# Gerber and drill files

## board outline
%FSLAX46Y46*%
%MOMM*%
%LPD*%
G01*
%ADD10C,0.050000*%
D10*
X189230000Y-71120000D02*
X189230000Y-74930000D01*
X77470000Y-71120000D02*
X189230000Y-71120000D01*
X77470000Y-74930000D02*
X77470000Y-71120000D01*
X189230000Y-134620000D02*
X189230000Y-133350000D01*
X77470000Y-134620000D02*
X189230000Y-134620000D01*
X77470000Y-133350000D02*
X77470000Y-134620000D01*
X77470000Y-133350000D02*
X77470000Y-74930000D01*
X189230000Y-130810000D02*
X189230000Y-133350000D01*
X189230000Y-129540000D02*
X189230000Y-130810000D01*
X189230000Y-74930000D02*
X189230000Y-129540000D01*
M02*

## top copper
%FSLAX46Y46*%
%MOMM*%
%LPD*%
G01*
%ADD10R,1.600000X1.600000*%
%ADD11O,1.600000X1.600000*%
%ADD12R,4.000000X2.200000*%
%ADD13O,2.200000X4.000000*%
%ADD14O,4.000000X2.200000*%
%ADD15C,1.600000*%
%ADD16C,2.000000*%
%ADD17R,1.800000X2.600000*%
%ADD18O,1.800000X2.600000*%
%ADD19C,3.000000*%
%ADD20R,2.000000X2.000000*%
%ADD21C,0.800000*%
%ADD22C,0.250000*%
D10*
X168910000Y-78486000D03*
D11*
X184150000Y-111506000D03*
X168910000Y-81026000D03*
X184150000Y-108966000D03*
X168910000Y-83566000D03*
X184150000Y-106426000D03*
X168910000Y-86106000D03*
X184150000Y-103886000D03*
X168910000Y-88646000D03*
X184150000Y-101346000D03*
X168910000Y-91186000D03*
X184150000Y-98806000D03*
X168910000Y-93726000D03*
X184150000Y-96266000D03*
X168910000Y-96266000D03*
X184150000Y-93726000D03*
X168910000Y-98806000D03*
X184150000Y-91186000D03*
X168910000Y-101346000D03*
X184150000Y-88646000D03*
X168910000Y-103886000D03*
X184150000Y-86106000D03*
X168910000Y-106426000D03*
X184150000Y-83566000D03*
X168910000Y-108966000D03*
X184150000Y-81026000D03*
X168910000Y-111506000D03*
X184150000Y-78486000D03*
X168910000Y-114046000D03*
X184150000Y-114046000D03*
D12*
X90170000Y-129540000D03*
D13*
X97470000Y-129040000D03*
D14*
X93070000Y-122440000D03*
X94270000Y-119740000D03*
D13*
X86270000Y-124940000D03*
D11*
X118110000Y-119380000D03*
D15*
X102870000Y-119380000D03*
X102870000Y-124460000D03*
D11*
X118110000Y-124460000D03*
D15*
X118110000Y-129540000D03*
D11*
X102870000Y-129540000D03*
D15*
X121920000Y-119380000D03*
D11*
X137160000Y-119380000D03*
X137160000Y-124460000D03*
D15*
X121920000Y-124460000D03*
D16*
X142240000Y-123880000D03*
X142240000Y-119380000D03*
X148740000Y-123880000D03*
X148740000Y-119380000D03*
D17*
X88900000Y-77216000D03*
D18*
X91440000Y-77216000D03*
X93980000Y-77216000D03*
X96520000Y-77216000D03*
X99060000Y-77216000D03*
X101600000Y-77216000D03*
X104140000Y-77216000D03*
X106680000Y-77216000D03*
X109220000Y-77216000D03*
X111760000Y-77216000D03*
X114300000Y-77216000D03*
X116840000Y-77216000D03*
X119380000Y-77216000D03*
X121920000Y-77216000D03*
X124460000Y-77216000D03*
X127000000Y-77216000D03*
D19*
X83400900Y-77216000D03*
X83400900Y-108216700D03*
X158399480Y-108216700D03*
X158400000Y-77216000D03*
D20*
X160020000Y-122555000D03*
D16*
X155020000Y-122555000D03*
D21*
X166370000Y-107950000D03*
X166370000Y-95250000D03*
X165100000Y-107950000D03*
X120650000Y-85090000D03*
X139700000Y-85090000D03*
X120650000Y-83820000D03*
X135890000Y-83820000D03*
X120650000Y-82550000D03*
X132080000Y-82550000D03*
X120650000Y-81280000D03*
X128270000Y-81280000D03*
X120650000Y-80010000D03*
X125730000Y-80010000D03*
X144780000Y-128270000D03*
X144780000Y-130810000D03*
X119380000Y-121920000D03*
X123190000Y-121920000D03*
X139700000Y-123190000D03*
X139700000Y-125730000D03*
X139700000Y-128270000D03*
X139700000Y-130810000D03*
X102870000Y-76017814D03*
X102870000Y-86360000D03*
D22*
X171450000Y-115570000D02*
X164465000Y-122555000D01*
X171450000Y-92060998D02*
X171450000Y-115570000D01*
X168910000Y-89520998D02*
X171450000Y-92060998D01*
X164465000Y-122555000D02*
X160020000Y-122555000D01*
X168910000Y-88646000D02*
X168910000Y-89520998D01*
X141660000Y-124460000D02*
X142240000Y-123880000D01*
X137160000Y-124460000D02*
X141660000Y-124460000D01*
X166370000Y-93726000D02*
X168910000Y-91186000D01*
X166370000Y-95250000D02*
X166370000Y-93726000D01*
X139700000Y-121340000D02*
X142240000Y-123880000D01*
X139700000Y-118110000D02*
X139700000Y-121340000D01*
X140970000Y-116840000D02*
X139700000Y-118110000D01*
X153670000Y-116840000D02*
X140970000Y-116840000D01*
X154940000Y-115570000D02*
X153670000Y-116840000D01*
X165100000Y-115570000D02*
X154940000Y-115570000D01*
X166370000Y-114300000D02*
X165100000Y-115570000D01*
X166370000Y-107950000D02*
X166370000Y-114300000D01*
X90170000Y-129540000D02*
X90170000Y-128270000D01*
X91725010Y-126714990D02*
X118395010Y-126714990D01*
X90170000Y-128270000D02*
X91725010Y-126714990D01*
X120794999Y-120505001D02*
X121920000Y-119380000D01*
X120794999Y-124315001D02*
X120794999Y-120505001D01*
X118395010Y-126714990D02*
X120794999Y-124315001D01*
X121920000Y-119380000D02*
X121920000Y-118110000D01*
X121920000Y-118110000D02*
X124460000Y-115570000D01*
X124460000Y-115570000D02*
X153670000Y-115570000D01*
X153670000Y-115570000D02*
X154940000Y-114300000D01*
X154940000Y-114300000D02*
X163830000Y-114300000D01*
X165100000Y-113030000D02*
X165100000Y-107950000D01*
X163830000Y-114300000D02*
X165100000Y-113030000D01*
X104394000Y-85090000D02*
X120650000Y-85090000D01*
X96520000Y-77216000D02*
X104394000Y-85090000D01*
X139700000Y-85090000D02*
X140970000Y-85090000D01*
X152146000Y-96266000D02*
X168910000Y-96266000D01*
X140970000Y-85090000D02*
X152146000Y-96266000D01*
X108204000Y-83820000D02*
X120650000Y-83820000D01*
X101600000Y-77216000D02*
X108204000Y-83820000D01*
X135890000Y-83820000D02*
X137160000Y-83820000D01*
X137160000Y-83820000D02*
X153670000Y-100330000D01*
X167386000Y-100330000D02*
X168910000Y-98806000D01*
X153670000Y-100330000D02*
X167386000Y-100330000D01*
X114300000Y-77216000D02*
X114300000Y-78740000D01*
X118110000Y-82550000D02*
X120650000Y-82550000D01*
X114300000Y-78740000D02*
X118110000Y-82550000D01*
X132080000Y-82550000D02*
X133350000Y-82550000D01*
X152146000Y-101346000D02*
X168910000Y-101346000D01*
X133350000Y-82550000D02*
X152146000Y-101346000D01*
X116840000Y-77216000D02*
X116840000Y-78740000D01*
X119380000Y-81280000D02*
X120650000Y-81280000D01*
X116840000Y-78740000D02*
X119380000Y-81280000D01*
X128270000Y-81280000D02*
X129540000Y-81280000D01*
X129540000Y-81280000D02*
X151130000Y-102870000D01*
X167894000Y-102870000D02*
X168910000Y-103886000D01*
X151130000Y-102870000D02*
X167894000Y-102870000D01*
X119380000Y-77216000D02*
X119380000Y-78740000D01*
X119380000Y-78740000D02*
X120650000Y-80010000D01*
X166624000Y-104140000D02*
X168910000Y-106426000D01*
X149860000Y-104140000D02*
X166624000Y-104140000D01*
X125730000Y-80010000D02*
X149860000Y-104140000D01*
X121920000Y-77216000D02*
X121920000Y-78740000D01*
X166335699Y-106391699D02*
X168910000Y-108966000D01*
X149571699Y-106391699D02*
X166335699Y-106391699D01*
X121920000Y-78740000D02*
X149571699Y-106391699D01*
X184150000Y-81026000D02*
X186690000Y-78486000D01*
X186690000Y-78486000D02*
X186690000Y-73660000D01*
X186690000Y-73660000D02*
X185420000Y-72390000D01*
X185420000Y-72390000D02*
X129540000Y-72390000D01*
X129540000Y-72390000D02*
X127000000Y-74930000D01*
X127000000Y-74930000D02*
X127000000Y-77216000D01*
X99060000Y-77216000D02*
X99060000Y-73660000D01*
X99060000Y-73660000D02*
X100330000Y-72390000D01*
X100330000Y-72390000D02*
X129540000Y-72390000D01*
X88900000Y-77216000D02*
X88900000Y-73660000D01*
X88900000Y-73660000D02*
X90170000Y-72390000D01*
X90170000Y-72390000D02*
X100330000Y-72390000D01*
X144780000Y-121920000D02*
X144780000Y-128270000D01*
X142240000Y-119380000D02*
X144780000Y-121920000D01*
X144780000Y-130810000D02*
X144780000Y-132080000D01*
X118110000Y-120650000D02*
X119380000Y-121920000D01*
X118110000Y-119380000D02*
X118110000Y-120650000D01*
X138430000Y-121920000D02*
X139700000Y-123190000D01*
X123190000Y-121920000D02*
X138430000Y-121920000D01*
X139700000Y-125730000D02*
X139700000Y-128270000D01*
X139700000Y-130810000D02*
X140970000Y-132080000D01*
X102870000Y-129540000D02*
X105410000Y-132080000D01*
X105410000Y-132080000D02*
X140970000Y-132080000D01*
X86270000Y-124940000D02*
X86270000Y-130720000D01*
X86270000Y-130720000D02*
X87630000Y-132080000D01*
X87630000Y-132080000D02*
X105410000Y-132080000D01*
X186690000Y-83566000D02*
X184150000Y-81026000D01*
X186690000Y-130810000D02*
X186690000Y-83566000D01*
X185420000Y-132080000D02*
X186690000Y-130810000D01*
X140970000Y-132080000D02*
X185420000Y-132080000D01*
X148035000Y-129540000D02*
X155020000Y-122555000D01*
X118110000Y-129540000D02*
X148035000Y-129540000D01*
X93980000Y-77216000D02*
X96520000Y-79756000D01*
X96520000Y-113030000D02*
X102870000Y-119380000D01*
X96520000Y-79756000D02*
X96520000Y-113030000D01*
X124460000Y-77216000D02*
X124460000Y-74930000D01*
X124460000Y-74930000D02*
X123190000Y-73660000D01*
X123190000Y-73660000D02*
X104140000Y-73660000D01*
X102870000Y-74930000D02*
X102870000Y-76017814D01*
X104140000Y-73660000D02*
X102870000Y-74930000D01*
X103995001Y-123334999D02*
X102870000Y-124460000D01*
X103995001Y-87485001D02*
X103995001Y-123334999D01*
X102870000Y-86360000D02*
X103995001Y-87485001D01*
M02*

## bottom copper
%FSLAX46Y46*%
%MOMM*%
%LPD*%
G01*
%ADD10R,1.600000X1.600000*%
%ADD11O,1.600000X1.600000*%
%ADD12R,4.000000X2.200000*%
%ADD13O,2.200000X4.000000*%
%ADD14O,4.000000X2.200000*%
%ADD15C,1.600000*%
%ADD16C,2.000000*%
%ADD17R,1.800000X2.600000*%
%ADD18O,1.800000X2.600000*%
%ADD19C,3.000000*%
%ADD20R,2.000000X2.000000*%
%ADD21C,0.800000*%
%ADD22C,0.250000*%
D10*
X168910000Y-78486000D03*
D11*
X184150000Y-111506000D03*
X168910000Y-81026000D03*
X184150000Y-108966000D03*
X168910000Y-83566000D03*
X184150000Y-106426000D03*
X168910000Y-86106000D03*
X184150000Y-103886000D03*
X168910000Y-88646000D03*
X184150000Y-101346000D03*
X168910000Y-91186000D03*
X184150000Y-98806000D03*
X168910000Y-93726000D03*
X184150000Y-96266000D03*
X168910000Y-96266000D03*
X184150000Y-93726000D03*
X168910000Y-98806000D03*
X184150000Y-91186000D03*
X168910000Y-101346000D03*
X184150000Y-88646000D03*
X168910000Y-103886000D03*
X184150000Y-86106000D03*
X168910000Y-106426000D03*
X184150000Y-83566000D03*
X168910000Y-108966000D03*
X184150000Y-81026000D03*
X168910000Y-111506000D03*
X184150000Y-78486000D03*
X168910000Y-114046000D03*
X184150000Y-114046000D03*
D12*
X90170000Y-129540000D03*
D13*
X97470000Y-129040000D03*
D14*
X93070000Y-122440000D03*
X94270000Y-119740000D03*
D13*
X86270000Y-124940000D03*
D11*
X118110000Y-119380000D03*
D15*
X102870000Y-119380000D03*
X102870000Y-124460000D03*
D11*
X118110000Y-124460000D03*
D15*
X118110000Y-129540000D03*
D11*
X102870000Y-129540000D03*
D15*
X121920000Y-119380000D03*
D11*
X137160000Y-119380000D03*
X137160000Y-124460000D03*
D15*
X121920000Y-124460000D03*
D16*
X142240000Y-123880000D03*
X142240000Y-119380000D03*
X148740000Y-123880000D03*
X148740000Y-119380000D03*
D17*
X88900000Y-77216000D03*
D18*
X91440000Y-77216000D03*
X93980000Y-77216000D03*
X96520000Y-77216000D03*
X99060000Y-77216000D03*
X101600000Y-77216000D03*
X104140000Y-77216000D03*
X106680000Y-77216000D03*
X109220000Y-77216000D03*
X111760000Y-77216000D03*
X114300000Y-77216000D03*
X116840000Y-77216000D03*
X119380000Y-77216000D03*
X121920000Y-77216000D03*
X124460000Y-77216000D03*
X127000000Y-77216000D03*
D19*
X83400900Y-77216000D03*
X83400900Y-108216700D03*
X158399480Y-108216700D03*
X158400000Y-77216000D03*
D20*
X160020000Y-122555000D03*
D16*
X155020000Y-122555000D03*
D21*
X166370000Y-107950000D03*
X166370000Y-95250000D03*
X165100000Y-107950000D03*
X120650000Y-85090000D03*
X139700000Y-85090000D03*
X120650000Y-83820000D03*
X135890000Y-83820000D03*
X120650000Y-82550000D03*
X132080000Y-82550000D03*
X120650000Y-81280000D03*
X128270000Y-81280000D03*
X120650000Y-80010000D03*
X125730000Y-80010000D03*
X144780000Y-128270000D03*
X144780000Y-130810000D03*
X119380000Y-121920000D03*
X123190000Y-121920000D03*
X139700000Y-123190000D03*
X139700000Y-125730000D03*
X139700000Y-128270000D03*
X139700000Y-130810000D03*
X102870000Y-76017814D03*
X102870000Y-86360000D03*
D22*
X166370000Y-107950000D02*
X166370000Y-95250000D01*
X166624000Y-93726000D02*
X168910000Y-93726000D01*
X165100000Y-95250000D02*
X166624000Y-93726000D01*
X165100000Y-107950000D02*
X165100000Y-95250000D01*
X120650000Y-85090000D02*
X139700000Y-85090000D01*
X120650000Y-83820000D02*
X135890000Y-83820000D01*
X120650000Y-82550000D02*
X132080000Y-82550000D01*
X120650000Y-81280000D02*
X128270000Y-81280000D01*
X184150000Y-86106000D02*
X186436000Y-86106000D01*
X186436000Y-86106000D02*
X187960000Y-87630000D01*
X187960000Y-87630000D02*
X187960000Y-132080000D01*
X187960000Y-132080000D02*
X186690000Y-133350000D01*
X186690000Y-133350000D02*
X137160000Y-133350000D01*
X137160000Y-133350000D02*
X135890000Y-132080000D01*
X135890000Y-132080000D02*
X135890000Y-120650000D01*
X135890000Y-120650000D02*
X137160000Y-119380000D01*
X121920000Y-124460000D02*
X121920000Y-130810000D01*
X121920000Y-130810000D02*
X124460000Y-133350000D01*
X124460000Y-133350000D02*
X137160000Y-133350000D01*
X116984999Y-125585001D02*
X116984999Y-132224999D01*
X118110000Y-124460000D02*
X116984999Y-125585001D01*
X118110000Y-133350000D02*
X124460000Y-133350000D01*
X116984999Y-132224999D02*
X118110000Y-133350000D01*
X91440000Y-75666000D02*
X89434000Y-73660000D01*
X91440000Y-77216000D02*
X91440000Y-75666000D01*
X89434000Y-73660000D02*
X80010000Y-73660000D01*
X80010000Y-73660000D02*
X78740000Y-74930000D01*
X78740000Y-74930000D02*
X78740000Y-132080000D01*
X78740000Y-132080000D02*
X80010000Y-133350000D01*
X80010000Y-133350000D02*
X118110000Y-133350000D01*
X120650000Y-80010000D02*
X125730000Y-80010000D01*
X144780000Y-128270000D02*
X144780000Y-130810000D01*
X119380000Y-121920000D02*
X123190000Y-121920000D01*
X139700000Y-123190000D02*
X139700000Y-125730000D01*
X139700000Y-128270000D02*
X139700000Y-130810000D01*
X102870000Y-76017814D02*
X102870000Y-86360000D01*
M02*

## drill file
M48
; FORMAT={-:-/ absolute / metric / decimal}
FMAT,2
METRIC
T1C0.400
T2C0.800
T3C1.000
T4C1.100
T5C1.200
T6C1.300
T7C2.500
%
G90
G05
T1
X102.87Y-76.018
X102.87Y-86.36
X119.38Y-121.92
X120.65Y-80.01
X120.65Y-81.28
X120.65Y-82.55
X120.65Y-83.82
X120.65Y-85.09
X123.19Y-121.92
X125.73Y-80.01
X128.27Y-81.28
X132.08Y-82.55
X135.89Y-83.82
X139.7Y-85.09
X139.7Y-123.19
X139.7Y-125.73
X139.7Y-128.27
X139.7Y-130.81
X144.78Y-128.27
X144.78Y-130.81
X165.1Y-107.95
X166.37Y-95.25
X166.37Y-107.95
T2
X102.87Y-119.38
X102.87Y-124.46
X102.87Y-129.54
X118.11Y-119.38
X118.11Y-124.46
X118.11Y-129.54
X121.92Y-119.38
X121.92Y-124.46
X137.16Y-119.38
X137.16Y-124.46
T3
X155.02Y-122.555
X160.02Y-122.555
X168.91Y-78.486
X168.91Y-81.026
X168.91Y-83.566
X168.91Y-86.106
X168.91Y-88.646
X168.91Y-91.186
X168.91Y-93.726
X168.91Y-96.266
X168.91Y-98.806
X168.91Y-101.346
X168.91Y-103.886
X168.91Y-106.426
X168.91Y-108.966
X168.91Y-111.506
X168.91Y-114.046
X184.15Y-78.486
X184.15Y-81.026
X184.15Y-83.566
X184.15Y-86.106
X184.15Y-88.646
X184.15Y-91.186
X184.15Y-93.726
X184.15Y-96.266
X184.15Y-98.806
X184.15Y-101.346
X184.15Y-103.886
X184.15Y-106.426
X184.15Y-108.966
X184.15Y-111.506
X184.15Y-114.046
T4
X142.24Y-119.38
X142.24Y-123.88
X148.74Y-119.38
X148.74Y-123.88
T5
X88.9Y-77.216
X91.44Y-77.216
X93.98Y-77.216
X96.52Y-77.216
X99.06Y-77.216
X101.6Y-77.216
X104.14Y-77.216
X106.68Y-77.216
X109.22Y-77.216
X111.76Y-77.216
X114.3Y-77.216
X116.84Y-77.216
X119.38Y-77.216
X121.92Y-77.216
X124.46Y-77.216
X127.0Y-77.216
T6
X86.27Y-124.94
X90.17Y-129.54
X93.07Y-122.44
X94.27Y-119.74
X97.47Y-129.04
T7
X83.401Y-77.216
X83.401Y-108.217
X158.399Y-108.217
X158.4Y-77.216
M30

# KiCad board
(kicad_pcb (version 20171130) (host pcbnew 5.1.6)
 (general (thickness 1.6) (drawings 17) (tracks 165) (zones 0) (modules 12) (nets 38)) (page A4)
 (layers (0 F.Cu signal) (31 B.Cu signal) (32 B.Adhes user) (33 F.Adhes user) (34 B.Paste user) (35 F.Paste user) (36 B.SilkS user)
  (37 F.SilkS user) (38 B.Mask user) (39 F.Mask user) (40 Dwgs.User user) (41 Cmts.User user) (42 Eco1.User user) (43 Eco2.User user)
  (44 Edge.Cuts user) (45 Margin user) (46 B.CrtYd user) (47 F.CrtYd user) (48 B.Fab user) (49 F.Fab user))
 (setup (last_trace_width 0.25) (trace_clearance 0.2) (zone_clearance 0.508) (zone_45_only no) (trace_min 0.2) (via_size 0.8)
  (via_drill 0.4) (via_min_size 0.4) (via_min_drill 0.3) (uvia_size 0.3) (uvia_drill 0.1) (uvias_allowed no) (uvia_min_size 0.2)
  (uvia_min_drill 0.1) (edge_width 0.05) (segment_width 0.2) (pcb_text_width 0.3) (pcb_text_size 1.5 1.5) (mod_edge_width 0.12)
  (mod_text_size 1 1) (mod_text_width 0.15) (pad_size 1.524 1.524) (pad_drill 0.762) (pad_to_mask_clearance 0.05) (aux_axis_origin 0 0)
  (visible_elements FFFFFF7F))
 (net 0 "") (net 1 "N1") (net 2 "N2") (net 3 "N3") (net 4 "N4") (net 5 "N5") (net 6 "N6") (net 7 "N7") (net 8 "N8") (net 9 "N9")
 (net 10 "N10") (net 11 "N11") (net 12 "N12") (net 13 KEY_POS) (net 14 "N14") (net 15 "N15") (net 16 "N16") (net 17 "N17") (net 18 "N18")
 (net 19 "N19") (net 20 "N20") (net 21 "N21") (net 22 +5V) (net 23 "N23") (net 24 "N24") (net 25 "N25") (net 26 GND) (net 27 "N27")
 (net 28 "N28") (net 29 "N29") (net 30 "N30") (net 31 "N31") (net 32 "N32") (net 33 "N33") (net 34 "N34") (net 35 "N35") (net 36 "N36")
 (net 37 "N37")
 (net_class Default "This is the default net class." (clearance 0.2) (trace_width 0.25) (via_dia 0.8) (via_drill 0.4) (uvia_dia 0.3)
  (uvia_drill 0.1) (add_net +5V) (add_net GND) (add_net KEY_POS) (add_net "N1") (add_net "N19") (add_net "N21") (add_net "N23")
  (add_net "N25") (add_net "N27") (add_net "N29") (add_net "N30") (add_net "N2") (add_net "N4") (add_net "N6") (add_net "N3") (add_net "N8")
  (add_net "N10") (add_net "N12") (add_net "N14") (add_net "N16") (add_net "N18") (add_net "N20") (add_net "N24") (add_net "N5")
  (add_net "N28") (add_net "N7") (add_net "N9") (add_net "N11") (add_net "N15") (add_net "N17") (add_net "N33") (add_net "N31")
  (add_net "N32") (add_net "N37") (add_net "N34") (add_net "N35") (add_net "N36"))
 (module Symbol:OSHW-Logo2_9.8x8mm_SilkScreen (layer F.Cu) (at 181.102 124.968)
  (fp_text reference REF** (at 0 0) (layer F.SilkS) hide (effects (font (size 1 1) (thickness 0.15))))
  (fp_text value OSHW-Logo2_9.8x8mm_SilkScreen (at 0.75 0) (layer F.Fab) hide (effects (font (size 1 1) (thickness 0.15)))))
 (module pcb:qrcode (layer F.Cu) (at 172.466 125.222)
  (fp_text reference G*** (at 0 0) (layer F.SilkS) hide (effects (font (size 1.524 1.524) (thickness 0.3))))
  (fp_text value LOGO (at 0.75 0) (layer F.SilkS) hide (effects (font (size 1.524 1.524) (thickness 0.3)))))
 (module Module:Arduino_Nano (layer F.Cu) (at 168.91 78.486)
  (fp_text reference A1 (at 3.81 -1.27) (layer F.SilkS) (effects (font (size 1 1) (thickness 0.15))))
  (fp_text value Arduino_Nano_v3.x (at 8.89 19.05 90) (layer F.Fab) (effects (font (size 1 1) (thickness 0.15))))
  (pad 1 thru_hole rect (at 0 0) (size 1.6 1.6) (drill 1) (layers *.Cu *.Mask) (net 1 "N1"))
  (pad 17 thru_hole oval (at 15.24 33.02) (size 1.6 1.6) (drill 1) (layers *.Cu *.Mask) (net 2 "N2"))
  (pad 2 thru_hole oval (at 0 2.54) (size 1.6 1.6) (drill 1) (layers *.Cu *.Mask) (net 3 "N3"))
  (pad 18 thru_hole oval (at 15.24 30.48) (size 1.6 1.6) (drill 1) (layers *.Cu *.Mask) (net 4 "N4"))
  (pad 3 thru_hole oval (at 0 5.08) (size 1.6 1.6) (drill 1) (layers *.Cu *.Mask) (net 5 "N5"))
  (pad 19 thru_hole oval (at 15.24 27.94) (size 1.6 1.6) (drill 1) (layers *.Cu *.Mask) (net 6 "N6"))
  (pad 4 thru_hole oval (at 0 7.62) (size 1.6 1.6) (drill 1) (layers *.Cu *.Mask) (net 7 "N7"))
  (pad 20 thru_hole oval (at 15.24 25.4) (size 1.6 1.6) (drill 1) (layers *.Cu *.Mask) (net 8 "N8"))
  (pad 5 thru_hole oval (at 0 10.16) (size 1.6 1.6) (drill 1) (layers *.Cu *.Mask) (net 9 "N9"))
  (pad 21 thru_hole oval (at 15.24 22.86) (size 1.6 1.6) (drill 1) (layers *.Cu *.Mask) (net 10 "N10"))
  (pad 6 thru_hole oval (at 0 12.7) (size 1.6 1.6) (drill 1) (layers *.Cu *.Mask) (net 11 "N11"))
  (pad 22 thru_hole oval (at 15.24 20.32) (size 1.6 1.6) (drill 1) (layers *.Cu *.Mask) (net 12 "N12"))
  (pad 7 thru_hole oval (at 0 15.24) (size 1.6 1.6) (drill 1) (layers *.Cu *.Mask) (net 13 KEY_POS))
  (pad 23 thru_hole oval (at 15.24 17.78) (size 1.6 1.6) (drill 1) (layers *.Cu *.Mask) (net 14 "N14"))
  (pad 8 thru_hole oval (at 0 17.78) (size 1.6 1.6) (drill 1) (layers *.Cu *.Mask) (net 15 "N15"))
  (pad 24 thru_hole oval (at 15.24 15.24) (size 1.6 1.6) (drill 1) (layers *.Cu *.Mask) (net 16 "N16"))
  (pad 9 thru_hole oval (at 0 20.32) (size 1.6 1.6) (drill 1) (layers *.Cu *.Mask) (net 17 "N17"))
  (pad 25 thru_hole oval (at 15.24 12.7) (size 1.6 1.6) (drill 1) (layers *.Cu *.Mask) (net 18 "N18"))
  (pad 10 thru_hole oval (at 0 22.86) (size 1.6 1.6) (drill 1) (layers *.Cu *.Mask) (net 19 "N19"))
  (pad 26 thru_hole oval (at 15.24 10.16) (size 1.6 1.6) (drill 1) (layers *.Cu *.Mask) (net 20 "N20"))
  (pad 11 thru_hole oval (at 0 25.4) (size 1.6 1.6) (drill 1) (layers *.Cu *.Mask) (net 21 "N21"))
  (pad 27 thru_hole oval (at 15.24 7.62) (size 1.6 1.6) (drill 1) (layers *.Cu *.Mask) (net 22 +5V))
  (pad 12 thru_hole oval (at 0 27.94) (size 1.6 1.6) (drill 1) (layers *.Cu *.Mask) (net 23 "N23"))
  (pad 28 thru_hole oval (at 15.24 5.08) (size 1.6 1.6) (drill 1) (layers *.Cu *.Mask) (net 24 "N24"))
  (pad 13 thru_hole oval (at 0 30.48) (size 1.6 1.6) (drill 1) (layers *.Cu *.Mask) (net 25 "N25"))
  (pad 29 thru_hole oval (at 15.24 2.54) (size 1.6 1.6) (drill 1) (layers *.Cu *.Mask) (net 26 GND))
  (pad 14 thru_hole oval (at 0 33.02) (size 1.6 1.6) (drill 1) (layers *.Cu *.Mask) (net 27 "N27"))
  (pad 30 thru_hole oval (at 15.24 0) (size 1.6 1.6) (drill 1) (layers *.Cu *.Mask) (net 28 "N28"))
  (pad 15 thru_hole oval (at 0 35.56) (size 1.6 1.6) (drill 1) (layers *.Cu *.Mask) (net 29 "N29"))
  (pad 16 thru_hole oval (at 15.24 35.56) (size 1.6 1.6) (drill 1) (layers *.Cu *.Mask) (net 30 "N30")))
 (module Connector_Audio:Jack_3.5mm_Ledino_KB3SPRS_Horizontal (layer F.Cu) (at 90.17 129.54)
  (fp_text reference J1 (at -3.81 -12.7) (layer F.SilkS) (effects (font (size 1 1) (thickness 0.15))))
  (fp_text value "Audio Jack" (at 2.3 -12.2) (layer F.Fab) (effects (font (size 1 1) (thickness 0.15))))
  (pad T thru_hole rect (at 0 0) (size 4 2.2) (drill 1.3) (layers *.Cu *.Mask) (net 13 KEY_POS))
  (pad TN thru_hole oval (at 7.3 -0.5 90) (size 4 2.2) (drill 1.3) (layers *.Cu *.Mask))
  (pad RN thru_hole oval (at 2.9 -7.1) (size 4 2.2) (drill 1.3) (layers *.Cu *.Mask))
  (pad R thru_hole oval (at 4.1 -9.8) (size 4 2.2) (drill 1.3) (layers *.Cu *.Mask))
  (pad S thru_hole oval (at -3.9 -4.6) (size 2.2 4) (drill 1.3) (layers *.Cu *.Mask) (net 26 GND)))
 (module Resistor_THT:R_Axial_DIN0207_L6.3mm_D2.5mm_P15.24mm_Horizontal (layer F.Cu) (at 102.87 119.38)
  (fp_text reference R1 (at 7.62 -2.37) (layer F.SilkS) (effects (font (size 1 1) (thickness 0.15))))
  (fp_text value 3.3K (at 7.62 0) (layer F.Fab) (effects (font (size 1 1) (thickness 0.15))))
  (pad 2 thru_hole oval (at 15.24 0) (size 1.6 1.6) (drill 0.8) (layers *.Cu *.Mask) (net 26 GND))
  (pad 1 thru_hole circle (at 0 0) (size 1.6 1.6) (drill 0.8) (layers *.Cu *.Mask) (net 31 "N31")))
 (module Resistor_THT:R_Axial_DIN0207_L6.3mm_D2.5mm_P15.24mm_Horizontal (layer F.Cu) (at 102.87 124.46)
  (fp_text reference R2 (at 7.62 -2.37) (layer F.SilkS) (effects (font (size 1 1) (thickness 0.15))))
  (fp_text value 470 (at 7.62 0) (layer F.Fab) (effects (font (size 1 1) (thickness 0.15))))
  (pad 1 thru_hole circle (at 0 0) (size 1.6 1.6) (drill 0.8) (layers *.Cu *.Mask) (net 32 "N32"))
  (pad 2 thru_hole oval (at 15.24 0) (size 1.6 1.6) (drill 0.8) (layers *.Cu *.Mask) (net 22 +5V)))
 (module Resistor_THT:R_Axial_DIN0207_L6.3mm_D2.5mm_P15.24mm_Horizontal (layer F.Cu) (at 118.11 129.54 180)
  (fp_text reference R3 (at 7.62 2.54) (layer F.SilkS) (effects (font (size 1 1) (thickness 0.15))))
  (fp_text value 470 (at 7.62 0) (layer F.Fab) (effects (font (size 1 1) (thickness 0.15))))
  (pad 1 thru_hole circle (at 0 0 180) (size 1.6 1.6) (drill 0.8) (layers *.Cu *.Mask) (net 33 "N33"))
  (pad 2 thru_hole oval (at 15.24 0 180) (size 1.6 1.6) (drill 0.8) (layers *.Cu *.Mask) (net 26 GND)))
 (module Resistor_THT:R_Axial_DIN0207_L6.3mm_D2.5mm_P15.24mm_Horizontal (layer F.Cu) (at 121.92 119.38)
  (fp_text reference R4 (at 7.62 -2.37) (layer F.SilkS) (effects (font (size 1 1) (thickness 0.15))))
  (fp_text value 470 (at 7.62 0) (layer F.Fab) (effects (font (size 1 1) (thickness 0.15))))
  (pad 1 thru_hole circle (at 0 0) (size 1.6 1.6) (drill 0.8) (layers *.Cu *.Mask) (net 13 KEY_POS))
  (pad 2 thru_hole oval (at 15.24 0) (size 1.6 1.6) (drill 0.8) (layers *.Cu *.Mask) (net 22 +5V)))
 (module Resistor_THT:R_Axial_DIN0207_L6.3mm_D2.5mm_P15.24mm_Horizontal (layer F.Cu) (at 121.92 124.46)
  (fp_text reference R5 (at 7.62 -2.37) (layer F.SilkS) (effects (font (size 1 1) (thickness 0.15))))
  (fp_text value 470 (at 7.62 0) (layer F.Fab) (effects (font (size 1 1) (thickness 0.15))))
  (pad 2 thru_hole oval (at 15.24 0) (size 1.6 1.6) (drill 0.8) (layers *.Cu *.Mask) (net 11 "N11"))
  (pad 1 thru_hole circle (at 0 0) (size 1.6 1.6) (drill 0.8) (layers *.Cu *.Mask) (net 22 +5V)))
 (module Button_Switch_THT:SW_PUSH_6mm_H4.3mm (layer F.Cu) (at 142.24 119.38)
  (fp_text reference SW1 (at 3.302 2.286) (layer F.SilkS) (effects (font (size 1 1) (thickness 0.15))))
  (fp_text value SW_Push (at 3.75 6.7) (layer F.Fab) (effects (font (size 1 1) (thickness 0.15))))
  (pad 2 thru_hole circle (at 0 4.5 90) (size 2 2) (drill 1.1) (layers *.Cu *.Mask) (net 11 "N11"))
  (pad 1 thru_hole circle (at 0 0 90) (size 2 2) (drill 1.1) (layers *.Cu *.Mask) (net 26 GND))
  (pad 2 thru_hole circle (at 6.5 4.5 90) (size 2 2) (drill 1.1) (layers *.Cu *.Mask) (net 11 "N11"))
  (pad 1 thru_hole circle (at 6.5 0 90) (size 2 2) (drill 1.1) (layers *.Cu *.Mask) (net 26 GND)))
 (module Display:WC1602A (layer F.Cu) (at 88.9 77.216)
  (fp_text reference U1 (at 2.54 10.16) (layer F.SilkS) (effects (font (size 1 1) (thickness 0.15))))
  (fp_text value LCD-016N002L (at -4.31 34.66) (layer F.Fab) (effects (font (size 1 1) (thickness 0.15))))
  (pad 1 thru_hole rect (at 0 0) (size 1.8 2.6) (drill 1.2) (layers *.Cu *.Mask) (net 26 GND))
  (pad 2 thru_hole oval (at 2.54 0) (size 1.8 2.6) (drill 1.2) (layers *.Cu *.Mask) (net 22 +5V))
  (pad 3 thru_hole oval (at 5.08 0) (size 1.8 2.6) (drill 1.2) (layers *.Cu *.Mask) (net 31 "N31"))
  (pad 4 thru_hole oval (at 7.62 0) (size 1.8 2.6) (drill 1.2) (layers *.Cu *.Mask) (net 15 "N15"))
  (pad 5 thru_hole oval (at 10.16 0) (size 1.8 2.6) (drill 1.2) (layers *.Cu *.Mask) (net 26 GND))
  (pad 6 thru_hole oval (at 12.7 0) (size 1.8 2.6) (drill 1.2) (layers *.Cu *.Mask) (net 17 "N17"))
  (pad 7 thru_hole oval (at 15.24 0) (size 1.8 2.6) (drill 1.2) (layers *.Cu *.Mask) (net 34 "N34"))
  (pad 8 thru_hole oval (at 17.78 0) (size 1.8 2.6) (drill 1.2) (layers *.Cu *.Mask) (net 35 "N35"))
  (pad 9 thru_hole oval (at 20.32 0) (size 1.8 2.6) (drill 1.2) (layers *.Cu *.Mask) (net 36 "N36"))
  (pad 10 thru_hole oval (at 22.86 0) (size 1.8 2.6) (drill 1.2) (layers *.Cu *.Mask) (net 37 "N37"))
  (pad 11 thru_hole oval (at 25.4 0) (size 1.8 2.6) (drill 1.2) (layers *.Cu *.Mask) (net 19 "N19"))
  (pad 12 thru_hole oval (at 27.94 0) (size 1.8 2.6) (drill 1.2) (layers *.Cu *.Mask) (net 21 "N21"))
  (pad 13 thru_hole oval (at 30.48 0) (size 1.8 2.6) (drill 1.2) (layers *.Cu *.Mask) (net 23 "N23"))
  (pad 14 thru_hole oval (at 33.02 0) (size 1.8 2.6) (drill 1.2) (layers *.Cu *.Mask) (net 25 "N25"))
  (pad 15 thru_hole oval (at 35.56 0) (size 1.8 2.6) (drill 1.2) (layers *.Cu *.Mask) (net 32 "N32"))
  (pad 16 thru_hole oval (at 38.1 0) (size 1.8 2.6) (drill 1.2) (layers *.Cu *.Mask) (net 26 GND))
  (pad "" thru_hole circle (at -5.4991 0) (size 3 3) (drill 2.5) (layers *.Cu *.Mask))
  (pad "" thru_hole circle (at -5.4991 31.0007) (size 3 3) (drill 2.5) (layers *.Cu *.Mask))
  (pad "" thru_hole circle (at 69.49948 31.0007) (size 3 3) (drill 2.5) (layers *.Cu *.Mask))
  (pad "" thru_hole circle (at 69.5 0) (size 3 3) (drill 2.5) (layers *.Cu *.Mask)))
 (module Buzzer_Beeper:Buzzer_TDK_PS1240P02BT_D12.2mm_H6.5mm (layer F.Cu) (at 160.02 122.555 180)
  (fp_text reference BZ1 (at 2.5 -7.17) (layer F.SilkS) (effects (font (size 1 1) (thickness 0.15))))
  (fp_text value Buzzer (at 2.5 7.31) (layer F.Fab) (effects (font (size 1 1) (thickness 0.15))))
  (pad 1 thru_hole rect (at 0 0 180) (size 2 2) (drill 1) (layers *.Cu *.Mask) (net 9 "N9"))
  (pad 2 thru_hole circle (at 5 0 180) (size 2 2) (drill 1) (layers *.Cu *.Mask) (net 33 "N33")))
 (gr_line (start 189.23 71.12) (end 189.23 74.93) (layer Edge.Cuts) (width 0.05))
 (gr_line (start 77.47 71.12) (end 189.23 71.12) (layer Edge.Cuts) (width 0.05))
 (gr_line (start 77.47 74.93) (end 77.47 71.12) (layer Edge.Cuts) (width 0.05))
 (gr_line (start 189.23 134.62) (end 189.23 133.35) (layer Edge.Cuts) (width 0.05))
 (gr_line (start 77.47 134.62) (end 189.23 134.62) (layer Edge.Cuts) (width 0.05))
 (gr_line (start 77.47 133.35) (end 77.47 134.62) (layer Edge.Cuts) (width 0.05))
 (gr_line (start 77.47 133.35) (end 77.47 74.93) (layer Edge.Cuts) (width 0.05))
 (gr_line (start 189.23 130.81) (end 189.23 133.35) (layer Edge.Cuts) (width 0.05))
 (gr_line (start 189.23 129.54) (end 189.23 130.81) (layer Edge.Cuts) (width 0.05))
 (gr_line (start 189.23 74.93) (end 189.23 129.54) (layer Edge.Cuts) (width 0.05))
 (segment (start 171.45 115.57) (end 164.465 122.555) (width 0.25) (layer F.Cu) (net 9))
 (segment (start 171.45 92.060998) (end 171.45 115.57) (width 0.25) (layer F.Cu) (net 9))
 (segment (start 168.91 89.520998) (end 171.45 92.060998) (width 0.25) (layer F.Cu) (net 9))
 (segment (start 164.465 122.555) (end 160.02 122.555) (width 0.25) (layer F.Cu) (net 9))
 (segment (start 168.91 88.646) (end 168.91 89.520998) (width 0.25) (layer F.Cu) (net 9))
 (segment (start 141.66 124.46) (end 142.24 123.88) (width 0.25) (layer F.Cu) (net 11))
 (segment (start 137.16 124.46) (end 141.66 124.46) (width 0.25) (layer F.Cu) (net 11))
 (via (at 166.37 107.95) (size 0.8) (drill 0.4) (layers F.Cu B.Cu) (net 11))
 (via (at 166.37 95.25) (size 0.8) (drill 0.4) (layers F.Cu B.Cu) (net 11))
 (segment (start 166.37 107.95) (end 166.37 95.25) (width 0.25) (layer B.Cu) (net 11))
 (segment (start 166.37 93.726) (end 168.91 91.186) (width 0.25) (layer F.Cu) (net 11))
 (segment (start 166.37 95.25) (end 166.37 93.726) (width 0.25) (layer F.Cu) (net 11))
 (segment (start 139.7 121.34) (end 142.24 123.88) (width 0.25) (layer F.Cu) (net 11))
 (segment (start 139.7 118.11) (end 139.7 121.34) (width 0.25) (layer F.Cu) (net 11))
 (segment (start 140.97 116.84) (end 139.7 118.11) (width 0.25) (layer F.Cu) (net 11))
 (segment (start 153.67 116.84) (end 140.97 116.84) (width 0.25) (layer F.Cu) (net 11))
 (segment (start 154.94 115.57) (end 153.67 116.84) (width 0.25) (layer F.Cu) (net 11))
 (segment (start 165.1 115.57) (end 154.94 115.57) (width 0.25) (layer F.Cu) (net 11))
 (segment (start 166.37 114.3) (end 165.1 115.57) (width 0.25) (layer F.Cu) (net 11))
 (segment (start 166.37 107.95) (end 166.37 114.3) (width 0.25) (layer F.Cu) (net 11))
 (segment (start 90.17 129.54) (end 90.17 128.27) (width 0.25) (layer F.Cu) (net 13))
 (segment (start 91.72501 126.71499) (end 118.39501 126.71499) (width 0.25) (layer F.Cu) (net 13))
 (segment (start 90.17 128.27) (end 91.72501 126.71499) (width 0.25) (layer F.Cu) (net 13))
 (segment (start 120.794999 120.505001) (end 121.92 119.38) (width 0.25) (layer F.Cu) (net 13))
 (segment (start 120.794999 124.315001) (end 120.794999 120.505001) (width 0.25) (layer F.Cu) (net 13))
 (segment (start 118.39501 126.71499) (end 120.794999 124.315001) (width 0.25) (layer F.Cu) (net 13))
 (segment (start 121.92 119.38) (end 121.92 118.11) (width 0.25) (layer F.Cu) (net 13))
 (segment (start 121.92 118.11) (end 124.46 115.57) (width 0.25) (layer F.Cu) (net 13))
 (segment (start 124.46 115.57) (end 153.67 115.57) (width 0.25) (layer F.Cu) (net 13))
 (segment (start 153.67 115.57) (end 154.94 114.3) (width 0.25) (layer F.Cu) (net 13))
 (segment (start 154.94 114.3) (end 163.83 114.3) (width 0.25) (layer F.Cu) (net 13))
 (via (at 165.1 107.95) (size 0.8) (drill 0.4) (layers F.Cu B.Cu) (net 13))
 (segment (start 165.1 113.03) (end 165.1 107.95) (width 0.25) (layer F.Cu) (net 13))
 (segment (start 163.83 114.3) (end 165.1 113.03) (width 0.25) (layer F.Cu) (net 13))
 (segment (start 166.624 93.726) (end 168.91 93.726) (width 0.25) (layer B.Cu) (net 13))
 (segment (start 165.1 95.25) (end 166.624 93.726) (width 0.25) (layer B.Cu) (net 13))
 (segment (start 165.1 107.95) (end 165.1 95.25) (width 0.25) (layer B.Cu) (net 13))
 (via (at 120.65 85.09) (size 0.8) (drill 0.4) (layers F.Cu B.Cu) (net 15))
 (segment (start 104.394 85.09) (end 120.65 85.09) (width 0.25) (layer F.Cu) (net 15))
 (segment (start 96.52 77.216) (end 104.394 85.09) (width 0.25) (layer F.Cu) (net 15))
 (via (at 139.7 85.09) (size 0.8) (drill 0.4) (layers F.Cu B.Cu) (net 15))
 (segment (start 120.65 85.09) (end 139.7 85.09) (width 0.25) (layer B.Cu) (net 15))
 (segment (start 139.7 85.09) (end 140.97 85.09) (width 0.25) (layer F.Cu) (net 15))
 (segment (start 152.146 96.266) (end 168.91 96.266) (width 0.25) (layer F.Cu) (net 15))
 (segment (start 140.97 85.09) (end 152.146 96.266) (width 0.25) (layer F.Cu) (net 15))
 (via (at 120.65 83.82) (size 0.8) (drill 0.4) (layers F.Cu B.Cu) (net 17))
 (segment (start 108.204 83.82) (end 120.65 83.82) (width 0.25) (layer F.Cu) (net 17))
 (segment (start 101.6 77.216) (end 108.204 83.82) (width 0.25) (layer F.Cu) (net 17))
 (via (at 135.89 83.82) (size 0.8) (drill 0.4) (layers F.Cu B.Cu) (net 17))
 (segment (start 120.65 83.82) (end 135.89 83.82) (width 0.25) (layer B.Cu) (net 17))
 (segment (start 135.89 83.82) (end 137.16 83.82) (width 0.25) (layer F.Cu) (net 17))
 (segment (start 137.16 83.82) (end 153.67 100.33) (width 0.25) (layer F.Cu) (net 17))
 (segment (start 167.386 100.33) (end 168.91 98.806) (width 0.25) (layer F.Cu) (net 17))
 (segment (start 153.67 100.33) (end 167.386 100.33) (width 0.25) (layer F.Cu) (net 17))
 (segment (start 114.3 77.216) (end 114.3 78.74) (width 0.25) (layer F.Cu) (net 19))
 (via (at 120.65 82.55) (size 0.8) (drill 0.4) (layers F.Cu B.Cu) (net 19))
 (segment (start 118.11 82.55) (end 120.65 82.55) (width 0.25) (layer F.Cu) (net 19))
 (segment (start 114.3 78.74) (end 118.11 82.55) (width 0.25) (layer F.Cu) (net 19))
 (via (at 132.08 82.55) (size 0.8) (drill 0.4) (layers F.Cu B.Cu) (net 19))
 (segment (start 120.65 82.55) (end 132.08 82.55) (width 0.25) (layer B.Cu) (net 19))
 (segment (start 132.08 82.55) (end 133.35 82.55) (width 0.25) (layer F.Cu) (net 19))
 (segment (start 152.146 101.346) (end 168.91 101.346) (width 0.25) (layer F.Cu) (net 19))
 (segment (start 133.35 82.55) (end 152.146 101.346) (width 0.25) (layer F.Cu) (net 19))
 (segment (start 116.84 77.216) (end 116.84 78.74) (width 0.25) (layer F.Cu) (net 21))
 (via (at 120.65 81.28) (size 0.8) (drill 0.4) (layers F.Cu B.Cu) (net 21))
 (segment (start 119.38 81.28) (end 120.65 81.28) (width 0.25) (layer F.Cu) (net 21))
 (segment (start 116.84 78.74) (end 119.38 81.28) (width 0.25) (layer F.Cu) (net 21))
 (via (at 128.27 81.28) (size 0.8) (drill 0.4) (layers F.Cu B.Cu) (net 21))
 (segment (start 120.65 81.28) (end 128.27 81.28) (width 0.25) (layer B.Cu) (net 21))
 (segment (start 128.27 81.28) (end 129.54 81.28) (width 0.25) (layer F.Cu) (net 21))
 (segment (start 129.54 81.28) (end 151.13 102.87) (width 0.25) (layer F.Cu) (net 21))
 (segment (start 167.894 102.87) (end 168.91 103.886) (width 0.25) (layer F.Cu) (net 21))
 (segment (start 151.13 102.87) (end 167.894 102.87) (width 0.25) (layer F.Cu) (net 21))
 (segment (start 184.15 86.106) (end 186.436 86.106) (width 0.25) (layer B.Cu) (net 22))
 (segment (start 186.436 86.106) (end 187.96 87.63) (width 0.25) (layer B.Cu) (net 22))
 (segment (start 187.96 87.63) (end 187.96 132.08) (width 0.25) (layer B.Cu) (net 22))
 (segment (start 187.96 132.08) (end 186.69 133.35) (width 0.25) (layer B.Cu) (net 22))
 (segment (start 186.69 133.35) (end 137.16 133.35) (width 0.25) (layer B.Cu) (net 22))
 (segment (start 137.16 133.35) (end 135.89 132.08) (width 0.25) (layer B.Cu) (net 22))
 (segment (start 135.89 132.08) (end 135.89 120.65) (width 0.25) (layer B.Cu) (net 22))
 (segment (start 135.89 120.65) (end 137.16 119.38) (width 0.25) (layer B.Cu) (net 22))
 (segment (start 121.92 124.46) (end 121.92 130.81) (width 0.25) (layer B.Cu) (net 22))
 (segment (start 121.92 130.81) (end 124.46 133.35) (width 0.25) (layer B.Cu) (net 22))
 (segment (start 124.46 133.35) (end 137.16 133.35) (width 0.25) (layer B.Cu) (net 22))
 (segment (start 116.984999 125.585001) (end 116.984999 132.224999) (width 0.25) (layer B.Cu) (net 22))
 (segment (start 118.11 124.46) (end 116.984999 125.585001) (width 0.25) (layer B.Cu) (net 22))
 (segment (start 118.11 133.35) (end 124.46 133.35) (width 0.25) (layer B.Cu) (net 22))
 (segment (start 116.984999 132.224999) (end 118.11 133.35) (width 0.25) (layer B.Cu) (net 22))
 (segment (start 91.44 75.666) (end 89.434 73.66) (width 0.25) (layer B.Cu) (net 22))
 (segment (start 91.44 77.216) (end 91.44 75.666) (width 0.25) (layer B.Cu) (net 22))
 (segment (start 89.434 73.66) (end 80.01 73.66) (width 0.25) (layer B.Cu) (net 22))
 (segment (start 80.01 73.66) (end 78.74 74.93) (width 0.25) (layer B.Cu) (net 22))
 (segment (start 78.74 74.93) (end 78.74 132.08) (width 0.25) (layer B.Cu) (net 22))
 (segment (start 78.74 132.08) (end 80.01 133.35) (width 0.25) (layer B.Cu) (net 22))
 (segment (start 80.01 133.35) (end 118.11 133.35) (width 0.25) (layer B.Cu) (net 22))
 (segment (start 119.38 77.216) (end 119.38 78.74) (width 0.25) (layer F.Cu) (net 23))
 (via (at 120.65 80.01) (size 0.8) (drill 0.4) (layers F.Cu B.Cu) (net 23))
 (segment (start 119.38 78.74) (end 120.65 80.01) (width 0.25) (layer F.Cu) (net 23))
 (via (at 125.73 80.01) (size 0.8) (drill 0.4) (layers F.Cu B.Cu) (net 23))
 (segment (start 120.65 80.01) (end 125.73 80.01) (width 0.25) (layer B.Cu) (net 23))
 (segment (start 166.624 104.14) (end 168.91 106.426) (width 0.25) (layer F.Cu) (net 23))
 (segment (start 149.86 104.14) (end 166.624 104.14) (width 0.25) (layer F.Cu) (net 23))
 (segment (start 125.73 80.01) (end 149.86 104.14) (width 0.25) (layer F.Cu) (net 23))
 (segment (start 121.92 77.216) (end 121.92 78.74) (width 0.25) (layer F.Cu) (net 25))
 (segment (start 166.335699 106.391699) (end 168.91 108.966) (width 0.25) (layer F.Cu) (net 25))
 (segment (start 149.571699 106.391699) (end 166.335699 106.391699) (width 0.25) (layer F.Cu) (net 25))
 (segment (start 121.92 78.74) (end 149.571699 106.391699) (width 0.25) (layer F.Cu) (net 25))
 (segment (start 184.15 81.026) (end 186.69 78.486) (width 0.25) (layer F.Cu) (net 26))
 (segment (start 186.69 78.486) (end 186.69 73.66) (width 0.25) (layer F.Cu) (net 26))
 (segment (start 186.69 73.66) (end 185.42 72.39) (width 0.25) (layer F.Cu) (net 26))
 (segment (start 185.42 72.39) (end 129.54 72.39) (width 0.25) (layer F.Cu) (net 26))
 (segment (start 129.54 72.39) (end 127 74.93) (width 0.25) (layer F.Cu) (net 26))
 (segment (start 127 74.93) (end 127 77.216) (width 0.25) (layer F.Cu) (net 26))
 (segment (start 99.06 77.216) (end 99.06 73.66) (width 0.25) (layer F.Cu) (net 26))
 (segment (start 99.06 73.66) (end 100.33 72.39) (width 0.25) (layer F.Cu) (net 26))
 (segment (start 100.33 72.39) (end 129.54 72.39) (width 0.25) (layer F.Cu) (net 26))
 (segment (start 88.9 77.216) (end 88.9 73.66) (width 0.25) (layer F.Cu) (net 26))
 (segment (start 88.9 73.66) (end 90.17 72.39) (width 0.25) (layer F.Cu) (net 26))
 (segment (start 90.17 72.39) (end 100.33 72.39) (width 0.25) (layer F.Cu) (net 26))
 (via (at 144.78 128.27) (size 0.8) (drill 0.4) (layers F.Cu B.Cu) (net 26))
 (segment (start 144.78 121.92) (end 144.78 128.27) (width 0.25) (layer F.Cu) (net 26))
 (segment (start 142.24 119.38) (end 144.78 121.92) (width 0.25) (layer F.Cu) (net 26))
 (via (at 144.78 130.81) (size 0.8) (drill 0.4) (layers F.Cu B.Cu) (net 26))
 (segment (start 144.78 128.27) (end 144.78 130.81) (width 0.25) (layer B.Cu) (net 26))
 (segment (start 144.78 130.81) (end 144.78 132.08) (width 0.25) (layer F.Cu) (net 26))
 (segment (start 118.11 120.65) (end 119.38 121.92) (width 0.25) (layer F.Cu) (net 26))
 (via (at 119.38 121.92) (size 0.8) (drill 0.4) (layers F.Cu B.Cu) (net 26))
 (segment (start 118.11 119.38) (end 118.11 120.65) (width 0.25) (layer F.Cu) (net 26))
 (via (at 123.19 121.92) (size 0.8) (drill 0.4) (layers F.Cu B.Cu) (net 26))
 (segment (start 119.38 121.92) (end 123.19 121.92) (width 0.25) (layer B.Cu) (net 26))
 (via (at 139.7 123.19) (size 0.8) (drill 0.4) (layers F.Cu B.Cu) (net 26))
 (segment (start 138.43 121.92) (end 139.7 123.19) (width 0.25) (layer F.Cu) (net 26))
 (segment (start 123.19 121.92) (end 138.43 121.92) (width 0.25) (layer F.Cu) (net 26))
 (via (at 139.7 125.73) (size 0.8) (drill 0.4) (layers F.Cu B.Cu) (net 26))
 (segment (start 139.7 123.19) (end 139.7 125.73) (width 0.25) (layer B.Cu) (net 26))
 (via (at 139.7 128.27) (size 0.8) (drill 0.4) (layers F.Cu B.Cu) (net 26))
 (segment (start 139.7 125.73) (end 139.7 128.27) (width 0.25) (layer F.Cu) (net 26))
 (via (at 139.7 130.81) (size 0.8) (drill 0.4) (layers F.Cu B.Cu) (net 26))
 (segment (start 139.7 128.27) (end 139.7 130.81) (width 0.25) (layer B.Cu) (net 26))
 (segment (start 139.7 130.81) (end 140.97 132.08) (width 0.25) (layer F.Cu) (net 26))
 (segment (start 102.87 129.54) (end 105.41 132.08) (width 0.25) (layer F.Cu) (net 26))
 (segment (start 105.41 132.08) (end 140.97 132.08) (width 0.25) (layer F.Cu) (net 26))
 (segment (start 86.27 124.94) (end 86.27 130.72) (width 0.25) (layer F.Cu) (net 26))
 (segment (start 86.27 130.72) (end 87.63 132.08) (width 0.25) (layer F.Cu) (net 26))
 (segment (start 87.63 132.08) (end 105.41 132.08) (width 0.25) (layer F.Cu) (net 26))
 (segment (start 186.69 83.566) (end 184.15 81.026) (width 0.25) (layer F.Cu) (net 26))
 (segment (start 186.69 130.81) (end 186.69 83.566) (width 0.25) (layer F.Cu) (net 26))
 (segment (start 185.42 132.08) (end 186.69 130.81) (width 0.25) (layer F.Cu) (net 26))
 (segment (start 140.97 132.08) (end 185.42 132.08) (width 0.25) (layer F.Cu) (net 26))
 (segment (start 148.035 129.54) (end 155.02 122.555) (width 0.25) (layer F.Cu) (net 33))
 (segment (start 118.11 129.54) (end 148.035 129.54) (width 0.25) (layer F.Cu) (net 33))
 (segment (start 93.98 77.216) (end 96.52 79.756) (width 0.25) (layer F.Cu) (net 31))
 (segment (start 96.52 113.03) (end 102.87 119.38) (width 0.25) (layer F.Cu) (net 31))
 (segment (start 96.52 79.756) (end 96.52 113.03) (width 0.25) (layer F.Cu) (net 31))
 (segment (start 124.46 77.216) (end 124.46 74.93) (width 0.25) (layer F.Cu) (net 32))
 (segment (start 124.46 74.93) (end 123.19 73.66) (width 0.25) (layer F.Cu) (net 32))
 (segment (start 123.19 73.66) (end 104.14 73.66) (width 0.25) (layer F.Cu) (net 32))
 (via (at 102.87 76.017814) (size 0.8) (drill 0.4) (layers F.Cu B.Cu) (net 32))
 (segment (start 102.87 74.93) (end 102.87 76.017814) (width 0.25) (layer F.Cu) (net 32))
 (segment (start 104.14 73.66) (end 102.87 74.93) (width 0.25) (layer F.Cu) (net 32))
 (via (at 102.87 86.36) (size 0.8) (drill 0.4) (layers F.Cu B.Cu) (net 32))
 (segment (start 102.87 76.017814) (end 102.87 86.36) (width 0.25) (layer B.Cu) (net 32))
 (segment (start 103.995001 123.334999) (end 102.87 124.46) (width 0.25) (layer F.Cu) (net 32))
 (segment (start 103.995001 87.485001) (end 103.995001 123.334999) (width 0.25) (layer F.Cu) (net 32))
 (segment (start 102.87 86.36) (end 103.995001 87.485001) (width 0.25) (layer F.Cu) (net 32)))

